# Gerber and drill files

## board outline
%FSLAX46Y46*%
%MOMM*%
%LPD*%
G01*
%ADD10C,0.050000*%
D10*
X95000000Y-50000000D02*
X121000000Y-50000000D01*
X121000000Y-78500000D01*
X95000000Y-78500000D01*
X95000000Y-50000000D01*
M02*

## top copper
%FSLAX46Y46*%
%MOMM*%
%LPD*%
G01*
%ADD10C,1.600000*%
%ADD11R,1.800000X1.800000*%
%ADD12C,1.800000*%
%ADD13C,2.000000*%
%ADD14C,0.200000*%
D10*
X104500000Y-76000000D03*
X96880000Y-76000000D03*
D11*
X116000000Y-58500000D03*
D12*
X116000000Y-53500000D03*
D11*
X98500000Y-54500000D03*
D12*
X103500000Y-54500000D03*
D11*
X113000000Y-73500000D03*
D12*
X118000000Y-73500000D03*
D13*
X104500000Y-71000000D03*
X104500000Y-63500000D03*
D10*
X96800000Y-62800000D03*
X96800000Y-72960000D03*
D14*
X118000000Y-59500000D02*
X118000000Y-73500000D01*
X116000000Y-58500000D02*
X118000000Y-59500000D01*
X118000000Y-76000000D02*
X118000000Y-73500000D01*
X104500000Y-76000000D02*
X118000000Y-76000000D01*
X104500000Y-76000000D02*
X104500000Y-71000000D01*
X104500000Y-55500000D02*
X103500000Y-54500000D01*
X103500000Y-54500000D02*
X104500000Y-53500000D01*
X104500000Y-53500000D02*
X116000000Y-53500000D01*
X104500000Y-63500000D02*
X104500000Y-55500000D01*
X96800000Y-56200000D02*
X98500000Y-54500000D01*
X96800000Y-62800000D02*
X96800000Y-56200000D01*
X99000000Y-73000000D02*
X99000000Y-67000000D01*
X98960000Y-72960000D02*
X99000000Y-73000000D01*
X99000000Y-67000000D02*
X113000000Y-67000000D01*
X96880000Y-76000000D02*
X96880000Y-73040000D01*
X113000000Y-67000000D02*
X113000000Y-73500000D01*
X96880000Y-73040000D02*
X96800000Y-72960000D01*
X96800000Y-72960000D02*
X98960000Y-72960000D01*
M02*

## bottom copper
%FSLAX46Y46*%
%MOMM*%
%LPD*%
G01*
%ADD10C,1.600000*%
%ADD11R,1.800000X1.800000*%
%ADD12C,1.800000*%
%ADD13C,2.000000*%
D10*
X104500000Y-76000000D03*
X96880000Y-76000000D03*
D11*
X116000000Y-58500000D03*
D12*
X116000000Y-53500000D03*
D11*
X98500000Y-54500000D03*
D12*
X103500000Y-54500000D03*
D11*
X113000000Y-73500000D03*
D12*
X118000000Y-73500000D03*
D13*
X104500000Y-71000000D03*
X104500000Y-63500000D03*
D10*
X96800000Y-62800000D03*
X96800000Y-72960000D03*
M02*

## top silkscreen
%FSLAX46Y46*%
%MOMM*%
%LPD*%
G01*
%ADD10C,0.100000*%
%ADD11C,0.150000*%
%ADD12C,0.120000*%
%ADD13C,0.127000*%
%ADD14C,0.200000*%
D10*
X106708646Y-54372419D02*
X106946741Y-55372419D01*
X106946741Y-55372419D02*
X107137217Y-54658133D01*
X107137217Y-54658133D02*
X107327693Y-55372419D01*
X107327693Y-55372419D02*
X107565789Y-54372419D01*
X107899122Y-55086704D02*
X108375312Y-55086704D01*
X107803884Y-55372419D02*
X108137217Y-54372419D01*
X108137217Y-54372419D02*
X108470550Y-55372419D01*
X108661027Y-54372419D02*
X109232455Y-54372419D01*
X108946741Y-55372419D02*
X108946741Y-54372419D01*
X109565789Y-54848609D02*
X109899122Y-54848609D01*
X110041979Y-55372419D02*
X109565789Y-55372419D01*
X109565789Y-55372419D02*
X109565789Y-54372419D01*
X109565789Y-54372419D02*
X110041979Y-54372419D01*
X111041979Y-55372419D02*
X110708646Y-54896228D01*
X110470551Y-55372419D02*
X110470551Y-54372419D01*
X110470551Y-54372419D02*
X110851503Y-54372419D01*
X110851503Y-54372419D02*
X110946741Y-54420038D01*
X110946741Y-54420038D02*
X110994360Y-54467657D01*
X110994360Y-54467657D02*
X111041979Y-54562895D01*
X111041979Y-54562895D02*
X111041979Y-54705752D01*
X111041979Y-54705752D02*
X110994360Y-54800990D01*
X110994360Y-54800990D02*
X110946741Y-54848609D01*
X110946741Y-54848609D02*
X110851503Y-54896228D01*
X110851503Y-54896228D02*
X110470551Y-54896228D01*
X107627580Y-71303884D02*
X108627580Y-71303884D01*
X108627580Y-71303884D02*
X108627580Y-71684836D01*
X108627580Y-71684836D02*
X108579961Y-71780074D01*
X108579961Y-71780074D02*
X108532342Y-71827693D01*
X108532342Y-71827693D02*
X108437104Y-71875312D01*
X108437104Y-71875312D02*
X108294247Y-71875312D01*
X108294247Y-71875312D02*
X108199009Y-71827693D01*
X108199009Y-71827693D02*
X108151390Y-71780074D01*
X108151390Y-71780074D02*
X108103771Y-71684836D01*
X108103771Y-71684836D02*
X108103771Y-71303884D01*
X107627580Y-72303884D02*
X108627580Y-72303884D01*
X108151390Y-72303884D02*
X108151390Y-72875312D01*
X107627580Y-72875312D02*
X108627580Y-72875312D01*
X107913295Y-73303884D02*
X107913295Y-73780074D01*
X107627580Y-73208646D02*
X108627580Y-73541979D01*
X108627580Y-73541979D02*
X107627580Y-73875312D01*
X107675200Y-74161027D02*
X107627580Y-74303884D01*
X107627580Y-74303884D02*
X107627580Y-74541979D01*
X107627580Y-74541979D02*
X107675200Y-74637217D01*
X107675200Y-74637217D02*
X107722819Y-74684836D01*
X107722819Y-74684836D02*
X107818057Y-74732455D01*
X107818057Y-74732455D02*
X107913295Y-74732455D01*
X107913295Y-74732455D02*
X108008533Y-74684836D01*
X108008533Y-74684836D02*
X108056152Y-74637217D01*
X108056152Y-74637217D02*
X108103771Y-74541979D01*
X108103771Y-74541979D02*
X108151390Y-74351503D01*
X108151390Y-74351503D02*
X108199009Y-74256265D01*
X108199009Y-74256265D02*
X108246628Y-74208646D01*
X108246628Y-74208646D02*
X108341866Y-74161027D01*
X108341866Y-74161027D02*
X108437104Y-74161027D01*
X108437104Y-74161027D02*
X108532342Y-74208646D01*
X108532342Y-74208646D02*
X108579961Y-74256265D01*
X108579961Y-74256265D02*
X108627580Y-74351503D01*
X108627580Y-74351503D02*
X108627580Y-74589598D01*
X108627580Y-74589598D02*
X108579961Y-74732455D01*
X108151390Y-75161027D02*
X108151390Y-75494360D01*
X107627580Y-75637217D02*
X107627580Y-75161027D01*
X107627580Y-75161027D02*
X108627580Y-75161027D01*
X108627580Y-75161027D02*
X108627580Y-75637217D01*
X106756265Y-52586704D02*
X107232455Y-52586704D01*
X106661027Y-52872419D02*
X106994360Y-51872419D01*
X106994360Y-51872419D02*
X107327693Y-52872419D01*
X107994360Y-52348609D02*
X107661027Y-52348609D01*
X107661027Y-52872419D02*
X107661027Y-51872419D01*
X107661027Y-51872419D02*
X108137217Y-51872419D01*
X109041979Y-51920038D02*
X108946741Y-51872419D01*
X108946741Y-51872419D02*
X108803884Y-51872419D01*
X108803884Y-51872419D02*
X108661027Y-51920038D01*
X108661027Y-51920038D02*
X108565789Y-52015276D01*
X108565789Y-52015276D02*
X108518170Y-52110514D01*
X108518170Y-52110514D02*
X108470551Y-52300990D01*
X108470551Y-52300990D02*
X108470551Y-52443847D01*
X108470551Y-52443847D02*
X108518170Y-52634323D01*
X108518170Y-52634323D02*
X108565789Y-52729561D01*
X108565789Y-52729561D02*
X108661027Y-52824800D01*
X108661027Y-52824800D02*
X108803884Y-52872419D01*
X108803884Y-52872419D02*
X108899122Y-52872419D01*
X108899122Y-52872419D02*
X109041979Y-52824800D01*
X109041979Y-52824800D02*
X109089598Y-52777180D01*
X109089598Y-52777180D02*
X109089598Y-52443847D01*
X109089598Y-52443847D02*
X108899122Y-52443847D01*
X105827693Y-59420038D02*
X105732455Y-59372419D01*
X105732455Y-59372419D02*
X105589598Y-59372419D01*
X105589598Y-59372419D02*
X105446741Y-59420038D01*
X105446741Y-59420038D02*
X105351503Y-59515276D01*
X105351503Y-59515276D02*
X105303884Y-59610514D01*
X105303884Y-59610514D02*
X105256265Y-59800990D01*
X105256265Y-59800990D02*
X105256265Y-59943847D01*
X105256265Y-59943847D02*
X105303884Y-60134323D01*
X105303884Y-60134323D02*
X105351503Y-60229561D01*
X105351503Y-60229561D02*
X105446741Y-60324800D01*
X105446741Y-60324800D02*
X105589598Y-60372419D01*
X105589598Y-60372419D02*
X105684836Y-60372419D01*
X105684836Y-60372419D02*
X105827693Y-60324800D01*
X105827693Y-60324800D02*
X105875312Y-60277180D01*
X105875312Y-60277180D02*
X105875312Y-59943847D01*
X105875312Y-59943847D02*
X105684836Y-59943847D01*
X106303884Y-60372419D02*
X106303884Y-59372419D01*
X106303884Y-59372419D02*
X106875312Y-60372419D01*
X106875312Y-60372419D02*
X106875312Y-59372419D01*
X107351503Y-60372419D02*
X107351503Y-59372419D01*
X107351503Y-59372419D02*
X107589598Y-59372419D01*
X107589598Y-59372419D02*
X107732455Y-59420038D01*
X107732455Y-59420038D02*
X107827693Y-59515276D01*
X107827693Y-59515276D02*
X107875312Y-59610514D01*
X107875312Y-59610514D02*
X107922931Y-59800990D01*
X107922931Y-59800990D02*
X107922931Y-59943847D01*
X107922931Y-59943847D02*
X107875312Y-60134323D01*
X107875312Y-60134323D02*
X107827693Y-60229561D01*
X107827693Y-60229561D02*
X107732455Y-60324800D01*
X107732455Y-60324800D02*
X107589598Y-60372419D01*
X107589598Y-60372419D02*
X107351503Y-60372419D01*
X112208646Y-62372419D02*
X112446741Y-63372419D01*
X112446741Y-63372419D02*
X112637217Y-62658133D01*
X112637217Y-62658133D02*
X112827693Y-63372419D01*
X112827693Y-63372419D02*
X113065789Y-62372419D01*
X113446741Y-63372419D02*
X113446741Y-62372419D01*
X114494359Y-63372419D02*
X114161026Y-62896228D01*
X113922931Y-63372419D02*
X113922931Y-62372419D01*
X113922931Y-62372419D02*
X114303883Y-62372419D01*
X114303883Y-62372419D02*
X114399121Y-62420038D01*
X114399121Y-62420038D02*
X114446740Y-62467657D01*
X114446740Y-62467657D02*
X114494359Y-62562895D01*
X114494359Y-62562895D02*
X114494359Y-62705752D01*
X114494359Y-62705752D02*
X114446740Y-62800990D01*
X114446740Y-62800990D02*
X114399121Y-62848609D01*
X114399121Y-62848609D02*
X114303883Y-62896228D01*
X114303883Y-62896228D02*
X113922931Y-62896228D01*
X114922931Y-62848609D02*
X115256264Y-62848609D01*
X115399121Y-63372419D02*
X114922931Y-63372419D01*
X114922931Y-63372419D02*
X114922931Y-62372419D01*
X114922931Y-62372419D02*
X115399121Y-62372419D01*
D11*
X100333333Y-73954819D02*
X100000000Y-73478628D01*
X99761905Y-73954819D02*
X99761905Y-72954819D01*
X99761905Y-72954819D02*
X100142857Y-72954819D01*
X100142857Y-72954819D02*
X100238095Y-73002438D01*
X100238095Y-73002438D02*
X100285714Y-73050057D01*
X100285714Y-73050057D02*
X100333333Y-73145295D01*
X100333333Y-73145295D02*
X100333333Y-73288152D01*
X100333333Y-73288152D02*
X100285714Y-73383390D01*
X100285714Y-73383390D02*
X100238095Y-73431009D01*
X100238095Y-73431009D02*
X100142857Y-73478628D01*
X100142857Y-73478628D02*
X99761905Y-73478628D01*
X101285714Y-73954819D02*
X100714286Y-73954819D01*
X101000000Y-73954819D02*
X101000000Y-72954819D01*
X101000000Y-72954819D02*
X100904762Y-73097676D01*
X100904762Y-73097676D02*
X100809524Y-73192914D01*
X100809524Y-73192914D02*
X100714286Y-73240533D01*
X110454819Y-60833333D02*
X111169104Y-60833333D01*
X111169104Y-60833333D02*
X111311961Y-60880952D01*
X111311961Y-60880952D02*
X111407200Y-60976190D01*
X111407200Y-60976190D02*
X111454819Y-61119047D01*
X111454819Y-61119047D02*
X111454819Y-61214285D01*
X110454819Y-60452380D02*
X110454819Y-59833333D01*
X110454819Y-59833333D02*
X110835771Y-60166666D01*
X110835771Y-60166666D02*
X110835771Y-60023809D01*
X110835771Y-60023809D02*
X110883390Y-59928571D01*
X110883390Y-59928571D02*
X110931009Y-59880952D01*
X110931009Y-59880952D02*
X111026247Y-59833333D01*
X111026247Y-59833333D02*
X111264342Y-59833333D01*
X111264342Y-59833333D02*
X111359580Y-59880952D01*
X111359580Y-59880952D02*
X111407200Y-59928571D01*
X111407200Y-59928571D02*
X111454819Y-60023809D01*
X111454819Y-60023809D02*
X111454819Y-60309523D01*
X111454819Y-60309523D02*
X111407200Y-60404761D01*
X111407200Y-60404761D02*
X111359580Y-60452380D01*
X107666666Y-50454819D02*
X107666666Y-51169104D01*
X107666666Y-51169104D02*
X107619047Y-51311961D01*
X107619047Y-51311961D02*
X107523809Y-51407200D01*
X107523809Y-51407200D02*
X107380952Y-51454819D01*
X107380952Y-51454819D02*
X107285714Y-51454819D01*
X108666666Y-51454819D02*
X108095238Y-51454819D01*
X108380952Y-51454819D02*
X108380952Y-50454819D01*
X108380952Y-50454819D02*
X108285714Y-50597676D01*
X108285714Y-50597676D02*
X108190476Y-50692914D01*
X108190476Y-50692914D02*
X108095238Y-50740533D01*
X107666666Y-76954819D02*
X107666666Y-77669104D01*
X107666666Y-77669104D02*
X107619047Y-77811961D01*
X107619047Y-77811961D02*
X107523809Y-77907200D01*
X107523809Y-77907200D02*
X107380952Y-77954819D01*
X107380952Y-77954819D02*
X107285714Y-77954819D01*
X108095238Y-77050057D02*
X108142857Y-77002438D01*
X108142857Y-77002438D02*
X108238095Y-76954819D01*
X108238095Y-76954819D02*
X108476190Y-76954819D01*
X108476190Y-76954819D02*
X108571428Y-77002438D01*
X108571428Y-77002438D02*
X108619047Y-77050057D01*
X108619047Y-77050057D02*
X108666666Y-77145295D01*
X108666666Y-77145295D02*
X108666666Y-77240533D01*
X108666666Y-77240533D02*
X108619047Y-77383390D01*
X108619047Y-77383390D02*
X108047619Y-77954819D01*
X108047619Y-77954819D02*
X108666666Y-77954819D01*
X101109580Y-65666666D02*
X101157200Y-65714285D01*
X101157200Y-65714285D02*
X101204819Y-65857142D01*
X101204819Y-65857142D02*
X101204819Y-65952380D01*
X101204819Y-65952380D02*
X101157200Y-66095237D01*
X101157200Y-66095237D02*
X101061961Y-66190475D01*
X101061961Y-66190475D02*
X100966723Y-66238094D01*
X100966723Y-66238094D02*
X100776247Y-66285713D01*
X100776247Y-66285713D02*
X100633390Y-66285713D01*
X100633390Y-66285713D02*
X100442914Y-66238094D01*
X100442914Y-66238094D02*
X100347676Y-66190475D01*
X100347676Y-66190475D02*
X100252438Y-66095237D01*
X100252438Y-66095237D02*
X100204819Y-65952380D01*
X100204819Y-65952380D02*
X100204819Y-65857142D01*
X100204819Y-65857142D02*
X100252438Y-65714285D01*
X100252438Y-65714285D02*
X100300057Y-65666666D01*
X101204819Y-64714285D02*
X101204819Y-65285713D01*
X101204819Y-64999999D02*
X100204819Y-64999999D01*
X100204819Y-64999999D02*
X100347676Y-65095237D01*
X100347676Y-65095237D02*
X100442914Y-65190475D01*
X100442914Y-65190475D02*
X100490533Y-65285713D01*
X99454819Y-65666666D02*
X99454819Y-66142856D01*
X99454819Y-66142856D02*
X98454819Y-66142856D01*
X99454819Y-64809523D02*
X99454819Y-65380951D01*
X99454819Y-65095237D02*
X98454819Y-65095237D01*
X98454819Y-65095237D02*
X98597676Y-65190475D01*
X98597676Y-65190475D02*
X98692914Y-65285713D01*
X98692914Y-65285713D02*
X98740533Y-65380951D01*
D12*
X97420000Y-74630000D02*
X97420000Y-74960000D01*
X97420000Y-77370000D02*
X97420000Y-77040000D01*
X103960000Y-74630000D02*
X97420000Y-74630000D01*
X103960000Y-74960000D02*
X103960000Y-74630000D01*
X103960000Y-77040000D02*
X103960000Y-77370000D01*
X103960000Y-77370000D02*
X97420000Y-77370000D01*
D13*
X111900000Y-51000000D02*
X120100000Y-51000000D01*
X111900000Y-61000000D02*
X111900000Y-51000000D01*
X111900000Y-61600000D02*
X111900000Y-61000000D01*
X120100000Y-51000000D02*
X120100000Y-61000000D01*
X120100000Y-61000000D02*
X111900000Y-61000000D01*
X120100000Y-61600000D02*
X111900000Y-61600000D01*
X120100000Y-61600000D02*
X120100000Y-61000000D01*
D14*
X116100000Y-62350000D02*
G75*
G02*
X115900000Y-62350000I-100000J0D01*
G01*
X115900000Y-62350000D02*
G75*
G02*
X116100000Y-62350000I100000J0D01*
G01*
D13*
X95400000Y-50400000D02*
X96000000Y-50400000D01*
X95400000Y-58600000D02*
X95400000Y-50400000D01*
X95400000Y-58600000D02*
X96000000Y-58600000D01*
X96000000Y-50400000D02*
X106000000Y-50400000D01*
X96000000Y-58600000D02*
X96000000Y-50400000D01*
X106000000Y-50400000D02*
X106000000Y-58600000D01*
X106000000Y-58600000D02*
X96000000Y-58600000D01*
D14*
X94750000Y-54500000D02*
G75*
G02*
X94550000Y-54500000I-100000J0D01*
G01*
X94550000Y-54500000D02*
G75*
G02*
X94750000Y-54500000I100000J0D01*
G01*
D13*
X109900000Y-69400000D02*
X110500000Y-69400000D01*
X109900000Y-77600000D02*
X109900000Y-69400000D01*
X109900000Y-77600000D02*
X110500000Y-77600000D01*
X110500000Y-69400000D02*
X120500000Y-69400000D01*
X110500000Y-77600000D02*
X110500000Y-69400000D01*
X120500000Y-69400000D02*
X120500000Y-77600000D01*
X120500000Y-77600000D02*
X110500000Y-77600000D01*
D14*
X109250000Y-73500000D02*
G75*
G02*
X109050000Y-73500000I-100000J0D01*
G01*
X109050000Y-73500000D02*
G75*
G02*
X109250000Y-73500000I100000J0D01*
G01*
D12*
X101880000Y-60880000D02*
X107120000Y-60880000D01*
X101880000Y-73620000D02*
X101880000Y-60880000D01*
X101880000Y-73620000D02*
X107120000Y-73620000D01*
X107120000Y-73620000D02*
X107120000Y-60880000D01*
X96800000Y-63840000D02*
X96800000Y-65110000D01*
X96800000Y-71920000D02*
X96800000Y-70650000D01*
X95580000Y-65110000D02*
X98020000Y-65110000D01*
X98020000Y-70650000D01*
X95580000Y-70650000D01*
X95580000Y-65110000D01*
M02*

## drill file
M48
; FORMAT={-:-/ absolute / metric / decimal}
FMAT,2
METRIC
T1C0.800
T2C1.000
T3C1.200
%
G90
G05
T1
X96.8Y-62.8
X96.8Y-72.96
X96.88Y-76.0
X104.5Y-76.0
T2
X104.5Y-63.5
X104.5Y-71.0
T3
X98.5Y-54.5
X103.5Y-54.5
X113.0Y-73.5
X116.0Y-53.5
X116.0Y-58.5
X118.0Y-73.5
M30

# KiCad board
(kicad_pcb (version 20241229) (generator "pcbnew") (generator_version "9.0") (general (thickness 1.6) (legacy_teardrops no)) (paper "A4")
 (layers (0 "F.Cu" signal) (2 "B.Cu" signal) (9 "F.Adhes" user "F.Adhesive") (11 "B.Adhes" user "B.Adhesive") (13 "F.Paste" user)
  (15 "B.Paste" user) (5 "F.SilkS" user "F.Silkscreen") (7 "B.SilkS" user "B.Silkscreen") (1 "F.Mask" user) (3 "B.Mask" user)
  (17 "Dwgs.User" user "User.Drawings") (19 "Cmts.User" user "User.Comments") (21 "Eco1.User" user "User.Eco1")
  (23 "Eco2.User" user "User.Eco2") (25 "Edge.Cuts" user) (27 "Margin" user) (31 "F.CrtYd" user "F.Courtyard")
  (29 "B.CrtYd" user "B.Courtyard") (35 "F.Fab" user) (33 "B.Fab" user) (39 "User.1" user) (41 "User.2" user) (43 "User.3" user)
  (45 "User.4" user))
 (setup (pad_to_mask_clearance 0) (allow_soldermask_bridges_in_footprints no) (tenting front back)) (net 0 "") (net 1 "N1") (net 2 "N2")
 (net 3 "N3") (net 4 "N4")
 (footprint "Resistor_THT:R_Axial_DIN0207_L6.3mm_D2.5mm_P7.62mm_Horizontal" (layer "F.Cu") (at 104.5 76 180)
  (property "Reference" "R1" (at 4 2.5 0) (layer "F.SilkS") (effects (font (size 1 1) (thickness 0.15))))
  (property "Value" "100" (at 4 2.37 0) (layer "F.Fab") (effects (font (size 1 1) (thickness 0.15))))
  (fp_line (start 7.08 1.37) (end 7.08 1.04) (stroke (width 0.12) (type solid)) (layer "F.SilkS"))
  (fp_line (start 7.08 -1.37) (end 7.08 -1.04) (stroke (width 0.12) (type solid)) (layer "F.SilkS"))
  (fp_line (start 0.54 1.37) (end 7.08 1.37) (stroke (width 0.12) (type solid)) (layer "F.SilkS"))
  (fp_line (start 0.54 1.04) (end 0.54 1.37) (stroke (width 0.12) (type solid)) (layer "F.SilkS"))
  (fp_line (start 0.54 -1.04) (end 0.54 -1.37) (stroke (width 0.12) (type solid)) (layer "F.SilkS"))
  (fp_line (start 0.54 -1.37) (end 7.08 -1.37) (stroke (width 0.12) (type solid)) (layer "F.SilkS"))
  (pad "1" thru_hole circle (at 0 0 180) (size 1.6 1.6) (drill 0.8) (layers "*.Cu" "*.Mask") (remove_unused_layers no) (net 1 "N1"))
  (pad "2" thru_hole circle (at 7.62 0 180) (size 1.6 1.6) (drill 0.8) (layers "*.Cu" "*.Mask") (remove_unused_layers no) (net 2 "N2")))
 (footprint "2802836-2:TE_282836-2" (layer "F.Cu") (at 116 56 90)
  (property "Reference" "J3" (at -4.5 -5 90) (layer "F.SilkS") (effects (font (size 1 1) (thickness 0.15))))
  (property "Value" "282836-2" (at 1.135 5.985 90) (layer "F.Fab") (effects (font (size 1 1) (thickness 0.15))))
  (fp_line (start 5 -4.1) (end 5 4.1) (stroke (width 0.127) (type solid)) (layer "F.SilkS"))
  (fp_line (start -5 -4.1) (end 5 -4.1) (stroke (width 0.127) (type solid)) (layer "F.SilkS"))
  (fp_line (start -5.6 -4.1) (end -5 -4.1) (stroke (width 0.127) (type solid)) (layer "F.SilkS"))
  (fp_line (start 5 4.1) (end -5 4.1) (stroke (width 0.127) (type solid)) (layer "F.SilkS"))
  (fp_line (start -5 4.1) (end -5 -4.1) (stroke (width 0.127) (type solid)) (layer "F.SilkS"))
  (fp_line (start -5.6 4.1) (end -5.6 -4.1) (stroke (width 0.127) (type solid)) (layer "F.SilkS"))
  (fp_line (start -5.6 4.1) (end -5 4.1) (stroke (width 0.127) (type solid)) (layer "F.SilkS"))
  (fp_circle (center -6.35 0) (end -6.25 0) (stroke (width 0.2) (type solid)) (fill no) (layer "F.SilkS"))
  (pad "1" thru_hole rect (at -2.5 0 90) (size 1.8 1.8) (drill 1.2) (layers "*.Cu" "*.Mask") (remove_unused_layers no) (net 1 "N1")
   (solder_mask_margin 0.102))
  (pad "2" thru_hole circle (at 2.5 0 90) (size 1.8 1.8) (drill 1.2) (layers "*.Cu" "*.Mask") (remove_unused_layers no) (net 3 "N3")
   (solder_mask_margin 0.102)))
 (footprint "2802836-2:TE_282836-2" (layer "F.Cu") (at 101 54.5)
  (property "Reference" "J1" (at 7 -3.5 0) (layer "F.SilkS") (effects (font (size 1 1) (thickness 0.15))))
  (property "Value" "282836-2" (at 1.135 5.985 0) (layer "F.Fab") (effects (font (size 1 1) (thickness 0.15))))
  (fp_line (start -5.6 -4.1) (end -5 -4.1) (stroke (width 0.127) (type solid)) (layer "F.SilkS"))
  (fp_line (start -5.6 4.1) (end -5.6 -4.1) (stroke (width 0.127) (type solid)) (layer "F.SilkS"))
  (fp_line (start -5.6 4.1) (end -5 4.1) (stroke (width 0.127) (type solid)) (layer "F.SilkS"))
  (fp_line (start -5 -4.1) (end 5 -4.1) (stroke (width 0.127) (type solid)) (layer "F.SilkS"))
  (fp_line (start -5 4.1) (end -5 -4.1) (stroke (width 0.127) (type solid)) (layer "F.SilkS"))
  (fp_line (start 5 -4.1) (end 5 4.1) (stroke (width 0.127) (type solid)) (layer "F.SilkS"))
  (fp_line (start 5 4.1) (end -5 4.1) (stroke (width 0.127) (type solid)) (layer "F.SilkS"))
  (fp_circle (center -6.35 0) (end -6.25 0) (stroke (width 0.2) (type solid)) (fill no) (layer "F.SilkS"))
  (pad "1" thru_hole rect (at -2.5 0) (size 1.8 1.8) (drill 1.2) (layers "*.Cu" "*.Mask") (remove_unused_layers no) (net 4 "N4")
   (solder_mask_margin 0.102))
  (pad "2" thru_hole circle (at 2.5 0) (size 1.8 1.8) (drill 1.2) (layers "*.Cu" "*.Mask") (remove_unused_layers no) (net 3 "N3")
   (solder_mask_margin 0.102)))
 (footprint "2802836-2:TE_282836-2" (layer "F.Cu") (at 115.5 73.5)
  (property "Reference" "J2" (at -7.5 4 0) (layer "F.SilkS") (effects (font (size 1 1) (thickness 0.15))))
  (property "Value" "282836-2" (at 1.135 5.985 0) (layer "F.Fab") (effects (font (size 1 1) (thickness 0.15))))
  (fp_line (start -5.6 -4.1) (end -5 -4.1) (stroke (width 0.127) (type solid)) (layer "F.SilkS"))
  (fp_line (start -5.6 4.1) (end -5.6 -4.1) (stroke (width 0.127) (type solid)) (layer "F.SilkS"))
  (fp_line (start -5.6 4.1) (end -5 4.1) (stroke (width 0.127) (type solid)) (layer "F.SilkS"))
  (fp_line (start -5 -4.1) (end 5 -4.1) (stroke (width 0.127) (type solid)) (layer "F.SilkS"))
  (fp_line (start -5 4.1) (end -5 -4.1) (stroke (width 0.127) (type solid)) (layer "F.SilkS"))
  (fp_line (start 5 -4.1) (end 5 4.1) (stroke (width 0.127) (type solid)) (layer "F.SilkS"))
  (fp_line (start 5 4.1) (end -5 4.1) (stroke (width 0.127) (type solid)) (layer "F.SilkS"))
  (fp_circle (center -6.35 0) (end -6.25 0) (stroke (width 0.2) (type solid)) (fill no) (layer "F.SilkS"))
  (pad "1" thru_hole rect (at -2.5 0) (size 1.8 1.8) (drill 1.2) (layers "*.Cu" "*.Mask") (remove_unused_layers no) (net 2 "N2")
   (solder_mask_margin 0.102))
  (pad "2" thru_hole circle (at 2.5 0) (size 1.8 1.8) (drill 1.2) (layers "*.Cu" "*.Mask") (remove_unused_layers no) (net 1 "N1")
   (solder_mask_margin 0.102)))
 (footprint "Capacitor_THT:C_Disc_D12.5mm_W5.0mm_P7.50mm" (layer "F.Cu") (at 104.5 71 90)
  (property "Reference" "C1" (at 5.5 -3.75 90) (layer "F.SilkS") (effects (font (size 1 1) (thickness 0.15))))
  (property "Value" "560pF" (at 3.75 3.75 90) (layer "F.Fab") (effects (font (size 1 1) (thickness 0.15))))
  (fp_line (start 10.12 -2.62) (end 10.12 2.62) (stroke (width 0.12) (type solid)) (layer "F.SilkS"))
  (fp_line (start -2.62 -2.62) (end 10.12 -2.62) (stroke (width 0.12) (type solid)) (layer "F.SilkS"))
  (fp_line (start -2.62 -2.62) (end -2.62 2.62) (stroke (width 0.12) (type solid)) (layer "F.SilkS"))
  (fp_line (start -2.62 2.62) (end 10.12 2.62) (stroke (width 0.12) (type solid)) (layer "F.SilkS"))
  (pad "1" thru_hole circle (at 0 0 90) (size 2 2) (drill 1) (layers "*.Cu" "*.Mask") (remove_unused_layers no) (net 1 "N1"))
  (pad "2" thru_hole circle (at 7.5 0 90) (size 2 2) (drill 1) (layers "*.Cu" "*.Mask") (remove_unused_layers no) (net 3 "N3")))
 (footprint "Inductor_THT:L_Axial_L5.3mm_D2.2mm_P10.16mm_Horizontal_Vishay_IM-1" (layer "F.Cu") (at 96.8 62.8 -90)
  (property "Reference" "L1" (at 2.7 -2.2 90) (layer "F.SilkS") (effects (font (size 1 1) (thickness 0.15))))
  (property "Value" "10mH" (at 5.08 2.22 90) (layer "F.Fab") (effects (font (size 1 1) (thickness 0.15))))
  (fp_line (start 1.04 0) (end 2.31 0) (stroke (width 0.12) (type solid)) (layer "F.SilkS"))
  (fp_line (start 9.12 0) (end 7.85 0) (stroke (width 0.12) (type solid)) (layer "F.SilkS"))
  (fp_rect (start 2.31 -1.22) (end 7.85 1.22) (stroke (width 0.12) (type solid)) (fill no) (layer "F.SilkS"))
  (pad "1" thru_hole circle (at 0 0 270) (size 1.6 1.6) (drill 0.8) (layers "*.Cu" "*.Mask") (remove_unused_layers no) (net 4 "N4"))
  (pad "2" thru_hole circle (at 10.16 0 270) (size 1.6 1.6) (drill 0.8) (layers "*.Cu" "*.Mask") (remove_unused_layers no) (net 2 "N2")))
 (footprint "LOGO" (layer "B.Cu") (at 113.5 67.5 180)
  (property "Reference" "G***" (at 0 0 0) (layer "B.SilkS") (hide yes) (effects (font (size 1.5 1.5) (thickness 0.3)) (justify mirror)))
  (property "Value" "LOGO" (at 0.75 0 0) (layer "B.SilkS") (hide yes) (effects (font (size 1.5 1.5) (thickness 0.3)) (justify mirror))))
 (gr_poly (pts (xy 95 50) (xy 121 50) (xy 121 78.5) (xy 95 78.5)) (stroke (width 0.05) (type solid)) (fill no) (layer "Edge.Cuts"))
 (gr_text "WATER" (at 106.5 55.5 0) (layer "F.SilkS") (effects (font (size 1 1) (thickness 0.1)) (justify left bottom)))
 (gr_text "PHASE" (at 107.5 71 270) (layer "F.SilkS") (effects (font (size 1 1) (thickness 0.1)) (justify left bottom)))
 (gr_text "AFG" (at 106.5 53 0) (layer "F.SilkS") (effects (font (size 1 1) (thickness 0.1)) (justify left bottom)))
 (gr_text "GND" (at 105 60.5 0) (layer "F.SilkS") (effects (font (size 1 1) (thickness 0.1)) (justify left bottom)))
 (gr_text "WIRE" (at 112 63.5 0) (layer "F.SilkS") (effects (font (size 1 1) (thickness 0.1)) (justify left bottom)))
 (segment (start 118 59.5) (end 118 73.5) (width 0.2) (layer "F.Cu") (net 1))
 (segment (start 116 58.5) (end 118 59.5) (width 0.2) (layer "F.Cu") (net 1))
 (segment (start 118 76) (end 118 73.5) (width 0.2) (layer "F.Cu") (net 1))
 (segment (start 104.5 76) (end 118 76) (width 0.2) (layer "F.Cu") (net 1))
 (segment (start 104.5 76) (end 104.5 71) (width 0.2) (layer "F.Cu") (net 1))
 (segment (start 104.5 55.5) (end 103.5 54.5) (width 0.2) (layer "F.Cu") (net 3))
 (segment (start 103.5 54.5) (end 104.5 53.5) (width 0.2) (layer "F.Cu") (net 3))
 (segment (start 104.5 53.5) (end 116 53.5) (width 0.2) (layer "F.Cu") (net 3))
 (segment (start 104.5 63.5) (end 104.5 55.5) (width 0.2) (layer "F.Cu") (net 3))
 (segment (start 96.8 56.2) (end 98.5 54.5) (width 0.2) (layer "F.Cu") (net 4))
 (segment (start 96.8 62.8) (end 96.8 56.2) (width 0.2) (layer "F.Cu") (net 4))
 (segment (start 99 73) (end 99 67) (width 0.2) (layer "F.Cu") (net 2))
 (segment (start 98.96 72.96) (end 99 73) (width 0.2) (layer "F.Cu") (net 2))
 (segment (start 99 67) (end 113 67) (width 0.2) (layer "F.Cu") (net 2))
 (segment (start 96.88 76) (end 96.88 73.04) (width 0.2) (layer "F.Cu") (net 2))
 (segment (start 113 67) (end 113 73.5) (width 0.2) (layer "F.Cu") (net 2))
 (segment (start 96.88 73.04) (end 96.8 72.96) (width 0.2) (layer "F.Cu") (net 2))
 (segment (start 96.8 72.96) (end 98.96 72.96) (width 0.2) (layer "F.Cu") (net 2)))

